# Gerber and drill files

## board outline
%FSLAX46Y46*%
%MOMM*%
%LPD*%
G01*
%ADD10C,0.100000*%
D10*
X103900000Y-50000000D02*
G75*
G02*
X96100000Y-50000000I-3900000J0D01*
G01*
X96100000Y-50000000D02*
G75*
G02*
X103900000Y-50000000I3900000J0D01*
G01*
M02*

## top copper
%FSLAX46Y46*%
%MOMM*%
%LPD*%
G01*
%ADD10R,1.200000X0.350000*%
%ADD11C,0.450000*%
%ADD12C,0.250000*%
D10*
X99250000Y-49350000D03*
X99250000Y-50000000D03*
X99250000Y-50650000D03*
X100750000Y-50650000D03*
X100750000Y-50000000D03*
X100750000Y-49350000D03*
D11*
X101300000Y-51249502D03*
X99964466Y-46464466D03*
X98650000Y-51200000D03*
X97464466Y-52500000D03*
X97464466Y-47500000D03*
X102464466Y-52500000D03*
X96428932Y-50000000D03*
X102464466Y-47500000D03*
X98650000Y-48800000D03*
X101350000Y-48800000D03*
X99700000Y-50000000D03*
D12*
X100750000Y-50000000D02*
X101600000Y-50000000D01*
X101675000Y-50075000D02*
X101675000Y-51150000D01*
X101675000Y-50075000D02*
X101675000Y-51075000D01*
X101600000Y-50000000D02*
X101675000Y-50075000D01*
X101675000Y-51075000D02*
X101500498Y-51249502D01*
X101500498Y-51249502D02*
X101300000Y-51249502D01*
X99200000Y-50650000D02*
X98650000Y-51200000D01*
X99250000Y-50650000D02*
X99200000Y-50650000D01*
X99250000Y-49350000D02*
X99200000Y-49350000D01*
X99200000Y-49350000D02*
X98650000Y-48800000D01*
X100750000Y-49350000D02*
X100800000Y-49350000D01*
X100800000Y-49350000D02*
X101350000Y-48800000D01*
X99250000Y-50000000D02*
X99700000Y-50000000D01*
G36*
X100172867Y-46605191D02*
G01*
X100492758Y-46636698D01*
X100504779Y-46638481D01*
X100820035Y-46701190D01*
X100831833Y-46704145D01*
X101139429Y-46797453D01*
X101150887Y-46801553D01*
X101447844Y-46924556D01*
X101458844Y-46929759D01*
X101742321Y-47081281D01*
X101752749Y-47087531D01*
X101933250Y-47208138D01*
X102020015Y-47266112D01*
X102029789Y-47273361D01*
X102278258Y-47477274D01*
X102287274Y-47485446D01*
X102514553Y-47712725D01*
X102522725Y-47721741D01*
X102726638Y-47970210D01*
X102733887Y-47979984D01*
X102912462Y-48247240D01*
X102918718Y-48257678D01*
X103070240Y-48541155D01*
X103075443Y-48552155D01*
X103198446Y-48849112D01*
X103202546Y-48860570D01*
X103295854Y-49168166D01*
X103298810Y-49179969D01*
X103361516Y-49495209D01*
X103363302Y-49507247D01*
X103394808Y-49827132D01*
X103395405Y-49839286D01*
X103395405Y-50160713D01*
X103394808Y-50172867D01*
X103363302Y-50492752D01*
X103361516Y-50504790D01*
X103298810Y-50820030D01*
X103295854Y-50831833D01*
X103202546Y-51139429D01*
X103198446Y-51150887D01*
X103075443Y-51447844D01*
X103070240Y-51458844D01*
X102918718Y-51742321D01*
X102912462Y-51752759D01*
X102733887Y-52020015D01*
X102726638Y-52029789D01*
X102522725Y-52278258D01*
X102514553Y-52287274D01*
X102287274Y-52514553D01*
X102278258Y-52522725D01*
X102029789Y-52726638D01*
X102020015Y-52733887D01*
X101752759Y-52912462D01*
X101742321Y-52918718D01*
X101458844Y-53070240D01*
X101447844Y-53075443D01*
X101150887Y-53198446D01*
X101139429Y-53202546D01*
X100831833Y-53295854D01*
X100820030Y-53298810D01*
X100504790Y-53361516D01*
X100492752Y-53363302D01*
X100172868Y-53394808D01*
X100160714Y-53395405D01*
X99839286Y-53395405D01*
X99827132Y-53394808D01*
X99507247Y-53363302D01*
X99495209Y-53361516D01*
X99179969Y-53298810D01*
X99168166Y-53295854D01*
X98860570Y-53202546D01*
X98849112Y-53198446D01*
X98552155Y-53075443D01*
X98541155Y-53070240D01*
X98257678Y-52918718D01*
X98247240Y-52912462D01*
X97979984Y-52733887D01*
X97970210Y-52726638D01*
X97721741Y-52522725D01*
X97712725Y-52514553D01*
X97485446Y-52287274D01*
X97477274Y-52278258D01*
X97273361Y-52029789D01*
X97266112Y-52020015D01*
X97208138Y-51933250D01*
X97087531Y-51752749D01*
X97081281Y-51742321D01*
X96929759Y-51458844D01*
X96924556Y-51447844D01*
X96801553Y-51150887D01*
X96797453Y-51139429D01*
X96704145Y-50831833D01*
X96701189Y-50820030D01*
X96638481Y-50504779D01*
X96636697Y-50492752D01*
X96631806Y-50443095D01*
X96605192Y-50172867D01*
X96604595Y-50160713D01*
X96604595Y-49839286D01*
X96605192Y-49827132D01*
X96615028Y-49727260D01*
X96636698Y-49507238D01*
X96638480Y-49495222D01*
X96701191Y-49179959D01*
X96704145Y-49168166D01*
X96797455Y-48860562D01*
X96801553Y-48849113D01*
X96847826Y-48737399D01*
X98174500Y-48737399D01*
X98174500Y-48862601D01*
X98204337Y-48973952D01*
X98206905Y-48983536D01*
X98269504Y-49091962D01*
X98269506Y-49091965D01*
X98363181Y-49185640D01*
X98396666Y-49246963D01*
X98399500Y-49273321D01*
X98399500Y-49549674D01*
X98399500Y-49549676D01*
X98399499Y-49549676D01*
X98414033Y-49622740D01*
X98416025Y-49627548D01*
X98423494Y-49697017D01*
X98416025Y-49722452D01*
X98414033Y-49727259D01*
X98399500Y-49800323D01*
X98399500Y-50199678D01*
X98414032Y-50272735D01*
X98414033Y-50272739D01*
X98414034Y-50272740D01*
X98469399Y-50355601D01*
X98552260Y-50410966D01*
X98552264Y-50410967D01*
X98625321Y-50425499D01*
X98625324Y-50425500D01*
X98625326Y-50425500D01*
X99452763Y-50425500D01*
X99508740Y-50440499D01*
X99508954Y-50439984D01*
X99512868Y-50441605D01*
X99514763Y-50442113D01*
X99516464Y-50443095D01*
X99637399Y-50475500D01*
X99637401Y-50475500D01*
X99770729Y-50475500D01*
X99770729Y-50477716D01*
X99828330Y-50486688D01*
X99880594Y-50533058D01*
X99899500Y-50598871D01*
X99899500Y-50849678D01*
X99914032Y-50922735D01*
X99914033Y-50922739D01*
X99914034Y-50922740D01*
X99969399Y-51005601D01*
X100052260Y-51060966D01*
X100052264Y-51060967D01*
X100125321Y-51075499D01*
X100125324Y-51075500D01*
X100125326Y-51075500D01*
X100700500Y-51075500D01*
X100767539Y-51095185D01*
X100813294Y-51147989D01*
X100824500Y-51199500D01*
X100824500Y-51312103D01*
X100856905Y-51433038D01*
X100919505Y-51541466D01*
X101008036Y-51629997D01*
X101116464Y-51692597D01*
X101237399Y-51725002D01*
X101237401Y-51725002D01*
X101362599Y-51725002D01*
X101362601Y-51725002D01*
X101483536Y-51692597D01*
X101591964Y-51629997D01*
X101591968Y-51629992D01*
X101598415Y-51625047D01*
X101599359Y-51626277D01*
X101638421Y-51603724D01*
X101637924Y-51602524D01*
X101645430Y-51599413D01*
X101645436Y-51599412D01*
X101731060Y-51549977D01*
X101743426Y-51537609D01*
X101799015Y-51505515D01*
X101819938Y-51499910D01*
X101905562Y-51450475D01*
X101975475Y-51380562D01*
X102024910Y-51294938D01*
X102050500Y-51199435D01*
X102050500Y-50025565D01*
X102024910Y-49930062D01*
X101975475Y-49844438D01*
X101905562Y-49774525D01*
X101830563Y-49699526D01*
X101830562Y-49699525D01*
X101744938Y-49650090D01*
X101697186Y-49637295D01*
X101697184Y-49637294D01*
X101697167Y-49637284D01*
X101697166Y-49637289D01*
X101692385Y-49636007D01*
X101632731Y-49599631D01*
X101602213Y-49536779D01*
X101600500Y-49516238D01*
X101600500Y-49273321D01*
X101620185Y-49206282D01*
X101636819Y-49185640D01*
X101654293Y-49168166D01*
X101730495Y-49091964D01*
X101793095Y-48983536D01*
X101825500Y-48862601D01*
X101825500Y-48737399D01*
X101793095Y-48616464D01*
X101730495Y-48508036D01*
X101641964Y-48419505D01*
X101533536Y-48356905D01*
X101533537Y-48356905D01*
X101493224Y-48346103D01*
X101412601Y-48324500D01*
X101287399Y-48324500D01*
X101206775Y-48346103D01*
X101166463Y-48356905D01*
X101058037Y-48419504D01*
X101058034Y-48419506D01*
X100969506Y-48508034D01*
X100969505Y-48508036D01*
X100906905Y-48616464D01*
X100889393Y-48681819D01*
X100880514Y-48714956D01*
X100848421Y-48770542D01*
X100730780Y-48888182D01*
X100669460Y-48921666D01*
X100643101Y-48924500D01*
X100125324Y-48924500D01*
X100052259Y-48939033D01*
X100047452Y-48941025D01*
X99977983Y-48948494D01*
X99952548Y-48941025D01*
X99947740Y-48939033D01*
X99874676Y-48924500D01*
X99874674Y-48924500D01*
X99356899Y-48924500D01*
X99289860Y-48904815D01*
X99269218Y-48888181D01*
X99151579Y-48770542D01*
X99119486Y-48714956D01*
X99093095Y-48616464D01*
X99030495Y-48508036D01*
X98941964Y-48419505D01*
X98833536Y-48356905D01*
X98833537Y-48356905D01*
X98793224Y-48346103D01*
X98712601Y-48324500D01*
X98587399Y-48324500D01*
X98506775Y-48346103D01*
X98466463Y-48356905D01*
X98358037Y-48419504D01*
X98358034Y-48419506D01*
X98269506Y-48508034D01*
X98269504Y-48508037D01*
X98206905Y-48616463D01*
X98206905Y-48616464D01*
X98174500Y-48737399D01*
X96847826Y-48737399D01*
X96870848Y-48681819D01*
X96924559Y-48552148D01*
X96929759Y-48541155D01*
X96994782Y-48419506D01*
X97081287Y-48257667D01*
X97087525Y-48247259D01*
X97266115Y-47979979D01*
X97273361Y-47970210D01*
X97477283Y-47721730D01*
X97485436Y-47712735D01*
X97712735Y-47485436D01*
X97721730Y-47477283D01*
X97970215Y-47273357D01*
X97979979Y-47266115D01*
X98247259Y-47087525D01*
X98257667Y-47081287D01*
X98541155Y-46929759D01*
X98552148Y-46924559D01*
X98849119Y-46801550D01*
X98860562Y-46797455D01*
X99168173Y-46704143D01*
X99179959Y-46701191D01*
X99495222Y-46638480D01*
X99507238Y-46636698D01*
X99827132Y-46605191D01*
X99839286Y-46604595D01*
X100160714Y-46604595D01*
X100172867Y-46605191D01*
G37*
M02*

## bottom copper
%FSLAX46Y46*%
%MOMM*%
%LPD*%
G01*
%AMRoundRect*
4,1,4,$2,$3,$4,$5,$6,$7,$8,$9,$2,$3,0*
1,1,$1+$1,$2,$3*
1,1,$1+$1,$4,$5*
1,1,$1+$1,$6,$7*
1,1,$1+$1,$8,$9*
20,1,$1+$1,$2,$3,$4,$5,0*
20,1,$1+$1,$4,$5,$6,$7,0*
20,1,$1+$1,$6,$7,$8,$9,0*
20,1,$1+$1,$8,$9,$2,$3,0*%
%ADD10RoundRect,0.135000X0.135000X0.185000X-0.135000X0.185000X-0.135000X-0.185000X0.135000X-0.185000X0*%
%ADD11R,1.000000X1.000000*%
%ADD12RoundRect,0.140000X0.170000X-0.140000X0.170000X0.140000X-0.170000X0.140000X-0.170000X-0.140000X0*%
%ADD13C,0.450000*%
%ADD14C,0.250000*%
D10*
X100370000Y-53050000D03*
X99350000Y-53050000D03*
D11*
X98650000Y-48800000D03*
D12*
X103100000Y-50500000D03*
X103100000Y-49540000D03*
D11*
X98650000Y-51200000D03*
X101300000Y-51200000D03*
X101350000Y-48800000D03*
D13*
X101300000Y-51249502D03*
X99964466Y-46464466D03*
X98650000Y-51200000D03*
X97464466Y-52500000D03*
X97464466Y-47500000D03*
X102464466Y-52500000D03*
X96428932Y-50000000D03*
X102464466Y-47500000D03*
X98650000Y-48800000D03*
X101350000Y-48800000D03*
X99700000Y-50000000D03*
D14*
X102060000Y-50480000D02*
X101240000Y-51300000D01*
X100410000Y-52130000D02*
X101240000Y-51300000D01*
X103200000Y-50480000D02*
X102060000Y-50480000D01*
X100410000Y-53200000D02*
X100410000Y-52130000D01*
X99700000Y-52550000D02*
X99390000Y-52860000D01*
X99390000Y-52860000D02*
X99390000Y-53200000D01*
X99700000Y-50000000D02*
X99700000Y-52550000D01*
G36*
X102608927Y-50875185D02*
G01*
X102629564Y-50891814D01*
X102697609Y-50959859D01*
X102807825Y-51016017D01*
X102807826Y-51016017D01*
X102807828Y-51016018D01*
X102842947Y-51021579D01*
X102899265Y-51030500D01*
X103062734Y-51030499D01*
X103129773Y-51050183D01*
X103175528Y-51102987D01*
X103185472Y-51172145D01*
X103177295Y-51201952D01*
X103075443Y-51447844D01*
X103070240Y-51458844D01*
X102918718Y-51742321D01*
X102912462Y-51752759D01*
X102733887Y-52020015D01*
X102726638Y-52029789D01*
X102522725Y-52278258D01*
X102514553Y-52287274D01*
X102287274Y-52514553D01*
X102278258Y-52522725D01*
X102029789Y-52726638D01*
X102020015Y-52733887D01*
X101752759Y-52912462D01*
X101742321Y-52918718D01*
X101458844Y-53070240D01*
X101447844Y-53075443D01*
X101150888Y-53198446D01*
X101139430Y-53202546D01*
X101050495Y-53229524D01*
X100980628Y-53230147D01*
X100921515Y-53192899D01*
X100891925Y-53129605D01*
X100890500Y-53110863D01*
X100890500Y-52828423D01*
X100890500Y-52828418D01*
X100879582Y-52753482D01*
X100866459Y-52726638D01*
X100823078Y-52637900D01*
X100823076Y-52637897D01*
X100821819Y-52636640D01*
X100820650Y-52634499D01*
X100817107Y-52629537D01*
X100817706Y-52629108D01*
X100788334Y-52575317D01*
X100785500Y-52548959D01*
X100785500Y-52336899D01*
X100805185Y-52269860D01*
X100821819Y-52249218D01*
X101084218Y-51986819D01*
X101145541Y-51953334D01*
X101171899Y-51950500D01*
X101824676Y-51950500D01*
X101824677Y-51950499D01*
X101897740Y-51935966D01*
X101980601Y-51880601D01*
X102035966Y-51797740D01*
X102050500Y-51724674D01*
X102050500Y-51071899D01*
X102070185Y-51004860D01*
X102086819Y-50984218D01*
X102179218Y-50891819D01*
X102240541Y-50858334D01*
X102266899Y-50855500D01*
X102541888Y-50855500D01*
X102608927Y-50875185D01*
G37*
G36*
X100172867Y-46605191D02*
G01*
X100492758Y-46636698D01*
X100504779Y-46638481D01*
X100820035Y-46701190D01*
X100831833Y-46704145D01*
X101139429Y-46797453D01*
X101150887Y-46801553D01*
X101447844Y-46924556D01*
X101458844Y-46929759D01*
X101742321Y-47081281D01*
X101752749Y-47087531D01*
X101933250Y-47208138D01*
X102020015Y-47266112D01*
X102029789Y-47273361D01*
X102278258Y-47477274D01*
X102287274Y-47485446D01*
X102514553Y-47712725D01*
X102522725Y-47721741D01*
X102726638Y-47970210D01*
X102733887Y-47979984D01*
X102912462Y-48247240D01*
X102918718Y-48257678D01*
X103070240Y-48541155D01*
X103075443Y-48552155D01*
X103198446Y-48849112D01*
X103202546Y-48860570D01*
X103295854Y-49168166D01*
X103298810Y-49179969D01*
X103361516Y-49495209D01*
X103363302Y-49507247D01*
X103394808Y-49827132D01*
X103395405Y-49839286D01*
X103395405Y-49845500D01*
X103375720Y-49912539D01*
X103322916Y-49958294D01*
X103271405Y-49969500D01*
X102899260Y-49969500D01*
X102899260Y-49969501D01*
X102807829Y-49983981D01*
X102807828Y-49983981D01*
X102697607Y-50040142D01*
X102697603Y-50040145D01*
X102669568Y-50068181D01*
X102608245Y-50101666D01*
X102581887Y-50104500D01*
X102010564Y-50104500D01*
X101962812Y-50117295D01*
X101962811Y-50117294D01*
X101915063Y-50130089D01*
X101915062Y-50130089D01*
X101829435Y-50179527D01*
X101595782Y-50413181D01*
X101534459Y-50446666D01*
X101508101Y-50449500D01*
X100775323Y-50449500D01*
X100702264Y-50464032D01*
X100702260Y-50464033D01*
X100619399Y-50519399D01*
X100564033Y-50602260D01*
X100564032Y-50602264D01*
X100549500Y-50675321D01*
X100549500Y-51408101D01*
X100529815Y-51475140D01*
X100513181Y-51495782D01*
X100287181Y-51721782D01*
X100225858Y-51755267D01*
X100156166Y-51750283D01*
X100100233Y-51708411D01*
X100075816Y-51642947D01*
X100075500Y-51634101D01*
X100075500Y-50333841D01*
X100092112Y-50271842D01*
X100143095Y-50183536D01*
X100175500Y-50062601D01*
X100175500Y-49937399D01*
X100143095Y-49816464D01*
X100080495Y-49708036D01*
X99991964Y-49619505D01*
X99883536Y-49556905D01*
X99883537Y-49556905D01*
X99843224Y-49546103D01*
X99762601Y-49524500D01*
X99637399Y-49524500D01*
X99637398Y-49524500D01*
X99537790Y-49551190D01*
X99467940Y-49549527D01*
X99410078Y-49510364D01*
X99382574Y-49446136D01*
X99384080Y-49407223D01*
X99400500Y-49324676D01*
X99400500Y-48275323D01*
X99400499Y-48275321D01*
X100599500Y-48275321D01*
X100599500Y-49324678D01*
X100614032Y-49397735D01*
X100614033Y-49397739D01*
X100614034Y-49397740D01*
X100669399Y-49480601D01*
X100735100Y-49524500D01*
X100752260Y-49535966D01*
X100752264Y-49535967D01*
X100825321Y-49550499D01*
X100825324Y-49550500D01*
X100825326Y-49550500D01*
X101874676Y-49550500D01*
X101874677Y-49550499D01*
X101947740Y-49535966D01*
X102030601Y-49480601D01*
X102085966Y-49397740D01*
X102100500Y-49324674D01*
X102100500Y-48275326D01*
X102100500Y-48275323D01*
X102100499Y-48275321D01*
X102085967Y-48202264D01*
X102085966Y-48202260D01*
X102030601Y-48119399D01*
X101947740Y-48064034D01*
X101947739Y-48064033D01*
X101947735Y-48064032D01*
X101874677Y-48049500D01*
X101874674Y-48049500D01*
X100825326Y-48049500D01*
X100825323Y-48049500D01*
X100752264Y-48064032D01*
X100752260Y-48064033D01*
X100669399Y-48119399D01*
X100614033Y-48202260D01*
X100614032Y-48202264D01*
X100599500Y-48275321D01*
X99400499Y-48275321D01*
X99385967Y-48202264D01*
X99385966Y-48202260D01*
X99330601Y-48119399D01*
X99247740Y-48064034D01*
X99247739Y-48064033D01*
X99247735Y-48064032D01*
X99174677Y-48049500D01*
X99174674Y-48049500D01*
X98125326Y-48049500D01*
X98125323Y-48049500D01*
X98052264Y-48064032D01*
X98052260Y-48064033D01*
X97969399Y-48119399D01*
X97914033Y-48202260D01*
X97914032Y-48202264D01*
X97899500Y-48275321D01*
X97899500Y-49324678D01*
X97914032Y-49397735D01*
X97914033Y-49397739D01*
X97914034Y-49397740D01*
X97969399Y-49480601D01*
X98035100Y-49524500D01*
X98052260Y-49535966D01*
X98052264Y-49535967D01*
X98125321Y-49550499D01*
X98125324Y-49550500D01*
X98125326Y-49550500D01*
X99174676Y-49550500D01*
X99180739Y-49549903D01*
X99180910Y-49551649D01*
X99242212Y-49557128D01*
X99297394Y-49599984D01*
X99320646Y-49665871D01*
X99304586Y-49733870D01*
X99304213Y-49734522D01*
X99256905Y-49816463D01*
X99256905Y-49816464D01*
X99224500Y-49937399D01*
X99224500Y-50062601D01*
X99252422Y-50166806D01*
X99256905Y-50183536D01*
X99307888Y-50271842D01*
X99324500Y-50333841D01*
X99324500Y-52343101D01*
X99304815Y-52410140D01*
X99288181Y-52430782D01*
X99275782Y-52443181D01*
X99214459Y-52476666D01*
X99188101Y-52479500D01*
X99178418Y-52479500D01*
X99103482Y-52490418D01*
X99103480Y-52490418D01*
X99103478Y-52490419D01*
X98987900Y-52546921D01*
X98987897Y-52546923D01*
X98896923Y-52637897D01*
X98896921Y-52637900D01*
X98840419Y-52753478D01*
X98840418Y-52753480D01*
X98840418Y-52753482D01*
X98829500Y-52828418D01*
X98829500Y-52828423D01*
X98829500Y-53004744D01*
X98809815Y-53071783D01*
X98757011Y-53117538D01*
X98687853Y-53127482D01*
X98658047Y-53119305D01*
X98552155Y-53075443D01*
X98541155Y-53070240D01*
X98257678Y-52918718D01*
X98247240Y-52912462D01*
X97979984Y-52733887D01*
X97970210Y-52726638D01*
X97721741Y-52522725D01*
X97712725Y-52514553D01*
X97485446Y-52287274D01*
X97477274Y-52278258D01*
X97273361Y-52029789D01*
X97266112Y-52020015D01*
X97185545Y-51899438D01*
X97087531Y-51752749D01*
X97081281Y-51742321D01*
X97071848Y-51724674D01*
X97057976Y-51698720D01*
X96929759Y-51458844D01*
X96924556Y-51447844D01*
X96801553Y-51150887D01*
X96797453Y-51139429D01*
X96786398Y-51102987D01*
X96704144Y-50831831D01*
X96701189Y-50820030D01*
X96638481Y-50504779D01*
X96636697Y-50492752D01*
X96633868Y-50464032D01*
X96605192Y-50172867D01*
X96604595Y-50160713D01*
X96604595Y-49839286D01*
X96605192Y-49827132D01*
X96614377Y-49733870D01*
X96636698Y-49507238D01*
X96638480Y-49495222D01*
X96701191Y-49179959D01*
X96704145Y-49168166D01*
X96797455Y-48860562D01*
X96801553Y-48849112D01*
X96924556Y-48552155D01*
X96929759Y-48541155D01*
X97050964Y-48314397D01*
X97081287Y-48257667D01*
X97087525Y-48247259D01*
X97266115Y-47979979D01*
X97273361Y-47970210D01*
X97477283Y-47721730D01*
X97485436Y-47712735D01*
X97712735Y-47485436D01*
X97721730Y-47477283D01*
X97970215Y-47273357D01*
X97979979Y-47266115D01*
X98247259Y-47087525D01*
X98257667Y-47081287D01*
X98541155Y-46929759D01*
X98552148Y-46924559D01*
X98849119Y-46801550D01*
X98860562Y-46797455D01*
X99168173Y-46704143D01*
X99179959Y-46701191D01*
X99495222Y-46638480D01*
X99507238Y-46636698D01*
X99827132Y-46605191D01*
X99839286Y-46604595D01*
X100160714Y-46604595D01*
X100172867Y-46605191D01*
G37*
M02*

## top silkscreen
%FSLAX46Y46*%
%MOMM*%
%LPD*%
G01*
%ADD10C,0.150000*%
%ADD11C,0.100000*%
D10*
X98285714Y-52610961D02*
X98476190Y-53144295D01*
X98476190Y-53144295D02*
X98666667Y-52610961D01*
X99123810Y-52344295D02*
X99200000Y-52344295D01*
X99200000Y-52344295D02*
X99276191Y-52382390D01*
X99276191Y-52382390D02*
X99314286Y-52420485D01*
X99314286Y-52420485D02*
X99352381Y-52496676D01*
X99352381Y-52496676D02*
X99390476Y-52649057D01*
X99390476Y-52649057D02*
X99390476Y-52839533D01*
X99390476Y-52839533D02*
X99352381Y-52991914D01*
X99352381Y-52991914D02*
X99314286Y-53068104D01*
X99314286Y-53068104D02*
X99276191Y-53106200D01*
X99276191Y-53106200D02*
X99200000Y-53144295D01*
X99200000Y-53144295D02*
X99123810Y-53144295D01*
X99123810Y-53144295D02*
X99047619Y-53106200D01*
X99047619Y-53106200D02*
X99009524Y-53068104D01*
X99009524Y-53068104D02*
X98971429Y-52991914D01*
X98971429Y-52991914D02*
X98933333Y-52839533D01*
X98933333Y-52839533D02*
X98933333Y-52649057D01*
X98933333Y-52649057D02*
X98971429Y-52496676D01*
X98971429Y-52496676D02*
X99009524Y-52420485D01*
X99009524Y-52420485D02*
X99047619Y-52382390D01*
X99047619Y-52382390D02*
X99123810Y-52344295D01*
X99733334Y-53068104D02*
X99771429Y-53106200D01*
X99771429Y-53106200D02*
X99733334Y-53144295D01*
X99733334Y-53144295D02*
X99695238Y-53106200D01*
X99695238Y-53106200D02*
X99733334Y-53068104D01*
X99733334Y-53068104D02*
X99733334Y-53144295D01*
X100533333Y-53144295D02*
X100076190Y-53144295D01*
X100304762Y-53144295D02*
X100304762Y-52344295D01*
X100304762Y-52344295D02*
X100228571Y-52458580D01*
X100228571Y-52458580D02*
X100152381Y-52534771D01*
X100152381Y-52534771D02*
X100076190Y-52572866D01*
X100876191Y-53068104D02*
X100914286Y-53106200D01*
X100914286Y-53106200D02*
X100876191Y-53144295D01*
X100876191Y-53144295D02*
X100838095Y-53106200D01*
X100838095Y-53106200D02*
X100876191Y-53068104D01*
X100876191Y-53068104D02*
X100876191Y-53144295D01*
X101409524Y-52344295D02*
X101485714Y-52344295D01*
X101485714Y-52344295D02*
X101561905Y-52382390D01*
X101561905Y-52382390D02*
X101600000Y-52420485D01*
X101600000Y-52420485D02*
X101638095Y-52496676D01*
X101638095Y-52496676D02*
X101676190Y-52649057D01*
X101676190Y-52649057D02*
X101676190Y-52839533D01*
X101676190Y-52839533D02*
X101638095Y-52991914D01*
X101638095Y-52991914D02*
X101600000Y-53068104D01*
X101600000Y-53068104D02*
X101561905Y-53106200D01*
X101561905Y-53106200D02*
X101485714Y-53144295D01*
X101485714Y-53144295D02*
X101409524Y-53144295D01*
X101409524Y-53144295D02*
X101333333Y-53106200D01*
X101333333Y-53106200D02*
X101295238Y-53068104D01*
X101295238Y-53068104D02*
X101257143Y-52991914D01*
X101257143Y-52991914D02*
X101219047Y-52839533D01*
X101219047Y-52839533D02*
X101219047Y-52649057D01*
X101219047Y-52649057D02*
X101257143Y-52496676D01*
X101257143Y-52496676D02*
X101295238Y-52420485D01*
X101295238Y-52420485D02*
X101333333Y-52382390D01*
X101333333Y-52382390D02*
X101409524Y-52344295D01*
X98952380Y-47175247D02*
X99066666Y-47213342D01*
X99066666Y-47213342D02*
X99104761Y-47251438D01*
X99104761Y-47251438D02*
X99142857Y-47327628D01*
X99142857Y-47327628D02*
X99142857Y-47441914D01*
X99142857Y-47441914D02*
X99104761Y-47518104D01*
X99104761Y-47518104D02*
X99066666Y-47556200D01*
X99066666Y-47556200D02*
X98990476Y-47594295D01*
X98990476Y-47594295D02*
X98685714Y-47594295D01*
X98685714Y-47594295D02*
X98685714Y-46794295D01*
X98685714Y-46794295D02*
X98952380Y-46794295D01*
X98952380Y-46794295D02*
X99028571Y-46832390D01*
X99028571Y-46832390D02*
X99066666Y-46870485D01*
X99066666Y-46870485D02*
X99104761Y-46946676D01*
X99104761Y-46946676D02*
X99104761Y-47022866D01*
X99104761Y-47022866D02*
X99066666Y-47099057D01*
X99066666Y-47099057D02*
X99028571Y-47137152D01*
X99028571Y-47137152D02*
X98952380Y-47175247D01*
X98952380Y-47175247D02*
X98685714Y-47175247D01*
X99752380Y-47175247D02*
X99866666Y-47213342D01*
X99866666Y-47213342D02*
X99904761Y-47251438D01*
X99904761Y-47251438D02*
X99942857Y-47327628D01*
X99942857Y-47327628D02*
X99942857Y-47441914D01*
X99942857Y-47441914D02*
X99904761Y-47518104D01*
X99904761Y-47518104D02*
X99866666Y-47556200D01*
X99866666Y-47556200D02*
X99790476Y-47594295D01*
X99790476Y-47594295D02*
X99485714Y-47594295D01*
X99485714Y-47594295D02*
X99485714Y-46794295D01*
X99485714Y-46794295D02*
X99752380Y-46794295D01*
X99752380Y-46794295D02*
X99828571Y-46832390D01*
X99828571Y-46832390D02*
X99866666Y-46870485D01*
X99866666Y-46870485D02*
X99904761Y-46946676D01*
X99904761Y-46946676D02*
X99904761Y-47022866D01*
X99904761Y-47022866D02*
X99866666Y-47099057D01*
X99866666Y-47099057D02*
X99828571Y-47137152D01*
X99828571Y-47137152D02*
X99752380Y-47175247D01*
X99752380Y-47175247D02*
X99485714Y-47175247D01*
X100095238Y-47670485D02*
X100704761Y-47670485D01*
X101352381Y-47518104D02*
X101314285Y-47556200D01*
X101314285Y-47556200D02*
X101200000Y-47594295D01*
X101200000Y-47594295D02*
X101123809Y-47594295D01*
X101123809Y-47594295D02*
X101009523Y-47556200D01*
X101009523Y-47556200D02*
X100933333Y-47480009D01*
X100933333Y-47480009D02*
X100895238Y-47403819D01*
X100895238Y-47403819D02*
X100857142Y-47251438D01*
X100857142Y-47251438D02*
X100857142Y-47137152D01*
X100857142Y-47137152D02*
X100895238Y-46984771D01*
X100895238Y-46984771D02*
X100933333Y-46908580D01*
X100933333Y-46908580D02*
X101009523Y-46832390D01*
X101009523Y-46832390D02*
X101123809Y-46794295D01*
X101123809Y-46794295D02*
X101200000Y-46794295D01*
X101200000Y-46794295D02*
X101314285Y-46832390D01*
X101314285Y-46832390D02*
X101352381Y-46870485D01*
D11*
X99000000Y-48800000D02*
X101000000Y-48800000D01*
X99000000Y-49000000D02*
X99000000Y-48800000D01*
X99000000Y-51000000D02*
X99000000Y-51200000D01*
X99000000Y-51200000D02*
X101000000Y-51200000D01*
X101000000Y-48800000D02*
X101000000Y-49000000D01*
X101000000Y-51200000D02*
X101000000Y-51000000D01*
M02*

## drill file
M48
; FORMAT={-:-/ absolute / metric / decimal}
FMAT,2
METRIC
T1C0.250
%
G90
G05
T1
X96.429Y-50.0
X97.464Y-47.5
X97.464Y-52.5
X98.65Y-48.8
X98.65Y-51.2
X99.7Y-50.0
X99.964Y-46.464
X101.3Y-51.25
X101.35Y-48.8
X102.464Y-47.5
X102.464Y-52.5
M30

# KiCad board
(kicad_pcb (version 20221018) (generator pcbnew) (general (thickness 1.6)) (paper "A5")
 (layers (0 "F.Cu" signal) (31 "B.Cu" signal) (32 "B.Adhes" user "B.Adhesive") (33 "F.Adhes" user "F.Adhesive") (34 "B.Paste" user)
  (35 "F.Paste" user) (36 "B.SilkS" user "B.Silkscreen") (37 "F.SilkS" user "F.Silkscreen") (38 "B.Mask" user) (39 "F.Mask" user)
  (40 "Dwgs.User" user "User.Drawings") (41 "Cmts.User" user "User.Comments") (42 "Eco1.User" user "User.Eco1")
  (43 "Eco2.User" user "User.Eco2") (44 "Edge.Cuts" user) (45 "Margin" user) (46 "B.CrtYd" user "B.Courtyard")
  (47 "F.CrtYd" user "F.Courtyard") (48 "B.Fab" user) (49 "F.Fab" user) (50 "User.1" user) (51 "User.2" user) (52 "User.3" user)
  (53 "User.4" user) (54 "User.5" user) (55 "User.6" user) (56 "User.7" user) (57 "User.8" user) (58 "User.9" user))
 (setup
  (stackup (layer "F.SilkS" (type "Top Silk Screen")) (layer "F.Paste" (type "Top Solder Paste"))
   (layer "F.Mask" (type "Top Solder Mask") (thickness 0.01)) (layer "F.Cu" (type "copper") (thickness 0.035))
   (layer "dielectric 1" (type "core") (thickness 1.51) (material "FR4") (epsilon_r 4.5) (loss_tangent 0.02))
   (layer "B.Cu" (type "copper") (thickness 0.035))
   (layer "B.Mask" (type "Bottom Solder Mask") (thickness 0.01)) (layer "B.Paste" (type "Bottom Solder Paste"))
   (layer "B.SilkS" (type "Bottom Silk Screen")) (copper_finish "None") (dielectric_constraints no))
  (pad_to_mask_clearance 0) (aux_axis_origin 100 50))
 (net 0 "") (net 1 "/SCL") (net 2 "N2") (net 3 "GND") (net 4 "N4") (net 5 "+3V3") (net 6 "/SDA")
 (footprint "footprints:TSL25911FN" (layer "F.Cu") (at 100 50)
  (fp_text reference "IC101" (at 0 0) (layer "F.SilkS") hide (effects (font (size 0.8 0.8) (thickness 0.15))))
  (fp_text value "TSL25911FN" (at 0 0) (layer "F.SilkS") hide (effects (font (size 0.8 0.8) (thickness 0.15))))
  (fp_line (start -1 -1.2) (end 1 -1.2) (stroke (width 0.1) (type solid)) (layer "F.SilkS"))
  (fp_line (start -1 -1) (end -1 -1.2) (stroke (width 0.1) (type solid)) (layer "F.SilkS"))
  (fp_line (start -1 1) (end -1 1.2) (stroke (width 0.1) (type solid)) (layer "F.SilkS"))
  (fp_line (start -1 1.2) (end 1 1.2) (stroke (width 0.1) (type solid)) (layer "F.SilkS"))
  (fp_line (start 1 -1.2) (end 1 -1) (stroke (width 0.1) (type solid)) (layer "F.SilkS"))
  (fp_line (start 1 1.2) (end 1 1) (stroke (width 0.1) (type solid)) (layer "F.SilkS"))
  (pad "1" smd rect (at -0.75 -0.65 90) (size 0.35 1.2) (layers "F.Cu" "F.Paste" "F.Mask") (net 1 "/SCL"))
  (pad "2" smd rect (at -0.75 0 90) (size 0.35 1.2) (layers "F.Cu" "F.Paste" "F.Mask") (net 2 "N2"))
  (pad "3" smd rect (at -0.75 0.65 90) (size 0.35 1.2) (layers "F.Cu" "F.Paste" "F.Mask") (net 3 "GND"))
  (pad "4" smd rect (at 0.75 0.65 90) (size 0.35 1.2) (layers "F.Cu" "F.Paste" "F.Mask") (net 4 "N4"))
  (pad "5" smd rect (at 0.75 0 90) (size 0.35 1.2) (layers "F.Cu" "F.Paste" "F.Mask") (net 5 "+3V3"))
  (pad "6" smd rect (at 0.75 -0.65 90) (size 0.35 1.2) (layers "F.Cu" "F.Paste" "F.Mask") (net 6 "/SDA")))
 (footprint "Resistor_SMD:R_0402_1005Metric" (layer "B.Cu") (at 99.86 53.05 180)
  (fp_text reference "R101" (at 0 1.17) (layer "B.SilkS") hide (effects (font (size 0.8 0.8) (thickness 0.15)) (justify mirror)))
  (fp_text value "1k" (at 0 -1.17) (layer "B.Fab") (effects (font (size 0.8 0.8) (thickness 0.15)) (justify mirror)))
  (pad "1" smd roundrect (at -0.51 0 180) (size 0.54 0.64) (layers "B.Cu" "B.Paste" "B.Mask") (roundrect_rratio 0.25) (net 5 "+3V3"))
  (pad "2" smd roundrect (at 0.51 0 180) (size 0.54 0.64) (layers "B.Cu" "B.Paste" "B.Mask") (roundrect_rratio 0.25) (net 2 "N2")))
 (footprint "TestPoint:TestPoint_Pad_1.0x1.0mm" (layer "B.Cu") (at 98.65 48.8 180)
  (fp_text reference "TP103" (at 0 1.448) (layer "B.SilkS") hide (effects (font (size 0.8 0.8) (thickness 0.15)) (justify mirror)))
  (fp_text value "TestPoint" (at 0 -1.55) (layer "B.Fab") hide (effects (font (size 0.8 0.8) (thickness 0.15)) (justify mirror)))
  (pad "1" smd rect (at 0 0 180) (size 1 1) (layers "B.Cu" "B.Mask") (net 1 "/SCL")))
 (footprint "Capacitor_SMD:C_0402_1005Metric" (layer "B.Cu") (at 103.1 50.02 90)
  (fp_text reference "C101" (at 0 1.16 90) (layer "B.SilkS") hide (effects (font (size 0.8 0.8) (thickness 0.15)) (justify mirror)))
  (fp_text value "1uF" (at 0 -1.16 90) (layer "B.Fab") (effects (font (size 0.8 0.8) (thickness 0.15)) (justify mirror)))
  (pad "1" smd roundrect (at -0.48 0 90) (size 0.56 0.62) (layers "B.Cu" "B.Paste" "B.Mask") (roundrect_rratio 0.25) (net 5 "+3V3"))
  (pad "2" smd roundrect (at 0.48 0 90) (size 0.56 0.62) (layers "B.Cu" "B.Paste" "B.Mask") (roundrect_rratio 0.25) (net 3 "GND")))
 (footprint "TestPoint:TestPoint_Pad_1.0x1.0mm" (layer "B.Cu") (at 98.65 51.2 180)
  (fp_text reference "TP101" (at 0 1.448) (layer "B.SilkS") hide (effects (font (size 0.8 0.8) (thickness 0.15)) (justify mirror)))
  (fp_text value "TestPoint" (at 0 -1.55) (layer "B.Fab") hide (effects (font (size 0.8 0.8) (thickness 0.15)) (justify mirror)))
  (pad "1" smd rect (at 0 0 180) (size 1 1) (layers "B.Cu" "B.Mask") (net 3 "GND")))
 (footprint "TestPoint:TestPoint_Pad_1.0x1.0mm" (layer "B.Cu") (at 101.3 51.2 180)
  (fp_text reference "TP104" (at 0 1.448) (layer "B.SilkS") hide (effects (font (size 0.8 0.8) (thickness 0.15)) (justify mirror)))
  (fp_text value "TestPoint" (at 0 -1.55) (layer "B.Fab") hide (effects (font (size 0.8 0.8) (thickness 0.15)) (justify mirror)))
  (pad "1" smd rect (at 0 0 180) (size 1 1) (layers "B.Cu" "B.Mask") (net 5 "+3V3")))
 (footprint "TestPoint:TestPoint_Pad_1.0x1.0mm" (layer "B.Cu") (at 101.35 48.8 180)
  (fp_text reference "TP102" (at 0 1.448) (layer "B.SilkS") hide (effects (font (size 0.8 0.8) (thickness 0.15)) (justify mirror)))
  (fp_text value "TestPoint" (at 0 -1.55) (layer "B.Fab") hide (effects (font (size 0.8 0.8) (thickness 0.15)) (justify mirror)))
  (pad "1" smd rect (at 0 0 180) (size 1 1) (layers "B.Cu" "B.Mask") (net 6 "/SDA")))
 (gr_circle (center 100 50) (end 103.9 50) (stroke (width 0.1) (type default)) (fill none) (layer "Edge.Cuts"))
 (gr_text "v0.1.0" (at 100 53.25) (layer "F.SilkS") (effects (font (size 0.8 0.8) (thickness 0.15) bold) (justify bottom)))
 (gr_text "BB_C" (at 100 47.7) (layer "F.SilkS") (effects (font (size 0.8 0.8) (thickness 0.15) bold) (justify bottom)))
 (segment (start 100.75 50) (end 101.6 50) (width 0.25) (layer "F.Cu") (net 5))
 (segment (start 101.675 50.075) (end 101.675 51.15) (width 0.25) (layer "F.Cu") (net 5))
 (segment (start 101.675 50.075) (end 101.675 51.075) (width 0.25) (layer "F.Cu") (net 5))
 (segment (start 101.6 50) (end 101.675 50.075) (width 0.25) (layer "F.Cu") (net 5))
 (segment (start 101.675 51.075) (end 101.500498 51.249502) (width 0.25) (layer "F.Cu") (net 5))
 (segment (start 101.500498 51.249502) (end 101.3 51.249502) (width 0.25) (layer "F.Cu") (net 5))
 (via (at 101.3 51.249502) (size 0.45) (drill 0.25) (layers "F.Cu" "B.Cu") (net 5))
 (segment (start 102.06 50.48) (end 101.24 51.3) (width 0.25) (layer "B.Cu") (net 5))
 (segment (start 100.41 52.13) (end 101.24 51.3) (width 0.25) (layer "B.Cu") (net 5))
 (segment (start 103.2 50.48) (end 102.06 50.48) (width 0.25) (layer "B.Cu") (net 5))
 (segment (start 100.41 53.2) (end 100.41 52.13) (width 0.25) (layer "B.Cu") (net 5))
 (segment (start 99.2 50.65) (end 98.65 51.2) (width 0.25) (layer "F.Cu") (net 3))
 (segment (start 99.25 50.65) (end 99.2 50.65) (width 0.25) (layer "F.Cu") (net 3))
 (via (at 99.964466 46.464466) (size 0.45) (drill 0.25) (layers "F.Cu" "B.Cu") (free) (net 3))
 (via (at 98.65 51.2) (size 0.45) (drill 0.25) (layers "F.Cu" "B.Cu") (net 3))
 (via (at 97.464466 52.5) (size 0.45) (drill 0.25) (layers "F.Cu" "B.Cu") (free) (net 3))
 (via (at 97.464466 47.5) (size 0.45) (drill 0.25) (layers "F.Cu" "B.Cu") (free) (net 3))
 (via (at 102.464466 52.5) (size 0.45) (drill 0.25) (layers "F.Cu" "B.Cu") (free) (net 3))
 (via (at 96.428932 50) (size 0.45) (drill 0.25) (layers "F.Cu" "B.Cu") (free) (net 3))
 (via (at 102.464466 47.5) (size 0.45) (drill 0.25) (layers "F.Cu" "B.Cu") (free) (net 3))
 (segment (start 99.25 49.35) (end 99.2 49.35) (width 0.25) (layer "F.Cu") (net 1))
 (segment (start 99.2 49.35) (end 98.65 48.8) (width 0.25) (layer "F.Cu") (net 1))
 (via (at 98.65 48.8) (size 0.45) (drill 0.25) (layers "F.Cu" "B.Cu") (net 1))
 (segment (start 100.75 49.35) (end 100.8 49.35) (width 0.25) (layer "F.Cu") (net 6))
 (segment (start 100.8 49.35) (end 101.35 48.8) (width 0.25) (layer "F.Cu") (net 6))
 (via (at 101.35 48.8) (size 0.45) (drill 0.25) (layers "F.Cu" "B.Cu") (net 6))
 (segment (start 99.25 50) (end 99.7 50) (width 0.25) (layer "F.Cu") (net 2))
 (via (at 99.7 50) (size 0.45) (drill 0.25) (layers "F.Cu" "B.Cu") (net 2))
 (segment (start 99.7 52.55) (end 99.39 52.86) (width 0.25) (layer "B.Cu") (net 2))
 (segment (start 99.39 52.86) (end 99.39 53.2) (width 0.25) (layer "B.Cu") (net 2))
 (segment (start 99.7 50) (end 99.7 52.55) (width 0.25) (layer "B.Cu") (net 2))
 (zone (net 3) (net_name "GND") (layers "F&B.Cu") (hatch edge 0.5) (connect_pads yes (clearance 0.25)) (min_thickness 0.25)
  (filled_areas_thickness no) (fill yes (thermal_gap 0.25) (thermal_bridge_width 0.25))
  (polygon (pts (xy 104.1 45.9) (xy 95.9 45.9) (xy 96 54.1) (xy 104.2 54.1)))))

